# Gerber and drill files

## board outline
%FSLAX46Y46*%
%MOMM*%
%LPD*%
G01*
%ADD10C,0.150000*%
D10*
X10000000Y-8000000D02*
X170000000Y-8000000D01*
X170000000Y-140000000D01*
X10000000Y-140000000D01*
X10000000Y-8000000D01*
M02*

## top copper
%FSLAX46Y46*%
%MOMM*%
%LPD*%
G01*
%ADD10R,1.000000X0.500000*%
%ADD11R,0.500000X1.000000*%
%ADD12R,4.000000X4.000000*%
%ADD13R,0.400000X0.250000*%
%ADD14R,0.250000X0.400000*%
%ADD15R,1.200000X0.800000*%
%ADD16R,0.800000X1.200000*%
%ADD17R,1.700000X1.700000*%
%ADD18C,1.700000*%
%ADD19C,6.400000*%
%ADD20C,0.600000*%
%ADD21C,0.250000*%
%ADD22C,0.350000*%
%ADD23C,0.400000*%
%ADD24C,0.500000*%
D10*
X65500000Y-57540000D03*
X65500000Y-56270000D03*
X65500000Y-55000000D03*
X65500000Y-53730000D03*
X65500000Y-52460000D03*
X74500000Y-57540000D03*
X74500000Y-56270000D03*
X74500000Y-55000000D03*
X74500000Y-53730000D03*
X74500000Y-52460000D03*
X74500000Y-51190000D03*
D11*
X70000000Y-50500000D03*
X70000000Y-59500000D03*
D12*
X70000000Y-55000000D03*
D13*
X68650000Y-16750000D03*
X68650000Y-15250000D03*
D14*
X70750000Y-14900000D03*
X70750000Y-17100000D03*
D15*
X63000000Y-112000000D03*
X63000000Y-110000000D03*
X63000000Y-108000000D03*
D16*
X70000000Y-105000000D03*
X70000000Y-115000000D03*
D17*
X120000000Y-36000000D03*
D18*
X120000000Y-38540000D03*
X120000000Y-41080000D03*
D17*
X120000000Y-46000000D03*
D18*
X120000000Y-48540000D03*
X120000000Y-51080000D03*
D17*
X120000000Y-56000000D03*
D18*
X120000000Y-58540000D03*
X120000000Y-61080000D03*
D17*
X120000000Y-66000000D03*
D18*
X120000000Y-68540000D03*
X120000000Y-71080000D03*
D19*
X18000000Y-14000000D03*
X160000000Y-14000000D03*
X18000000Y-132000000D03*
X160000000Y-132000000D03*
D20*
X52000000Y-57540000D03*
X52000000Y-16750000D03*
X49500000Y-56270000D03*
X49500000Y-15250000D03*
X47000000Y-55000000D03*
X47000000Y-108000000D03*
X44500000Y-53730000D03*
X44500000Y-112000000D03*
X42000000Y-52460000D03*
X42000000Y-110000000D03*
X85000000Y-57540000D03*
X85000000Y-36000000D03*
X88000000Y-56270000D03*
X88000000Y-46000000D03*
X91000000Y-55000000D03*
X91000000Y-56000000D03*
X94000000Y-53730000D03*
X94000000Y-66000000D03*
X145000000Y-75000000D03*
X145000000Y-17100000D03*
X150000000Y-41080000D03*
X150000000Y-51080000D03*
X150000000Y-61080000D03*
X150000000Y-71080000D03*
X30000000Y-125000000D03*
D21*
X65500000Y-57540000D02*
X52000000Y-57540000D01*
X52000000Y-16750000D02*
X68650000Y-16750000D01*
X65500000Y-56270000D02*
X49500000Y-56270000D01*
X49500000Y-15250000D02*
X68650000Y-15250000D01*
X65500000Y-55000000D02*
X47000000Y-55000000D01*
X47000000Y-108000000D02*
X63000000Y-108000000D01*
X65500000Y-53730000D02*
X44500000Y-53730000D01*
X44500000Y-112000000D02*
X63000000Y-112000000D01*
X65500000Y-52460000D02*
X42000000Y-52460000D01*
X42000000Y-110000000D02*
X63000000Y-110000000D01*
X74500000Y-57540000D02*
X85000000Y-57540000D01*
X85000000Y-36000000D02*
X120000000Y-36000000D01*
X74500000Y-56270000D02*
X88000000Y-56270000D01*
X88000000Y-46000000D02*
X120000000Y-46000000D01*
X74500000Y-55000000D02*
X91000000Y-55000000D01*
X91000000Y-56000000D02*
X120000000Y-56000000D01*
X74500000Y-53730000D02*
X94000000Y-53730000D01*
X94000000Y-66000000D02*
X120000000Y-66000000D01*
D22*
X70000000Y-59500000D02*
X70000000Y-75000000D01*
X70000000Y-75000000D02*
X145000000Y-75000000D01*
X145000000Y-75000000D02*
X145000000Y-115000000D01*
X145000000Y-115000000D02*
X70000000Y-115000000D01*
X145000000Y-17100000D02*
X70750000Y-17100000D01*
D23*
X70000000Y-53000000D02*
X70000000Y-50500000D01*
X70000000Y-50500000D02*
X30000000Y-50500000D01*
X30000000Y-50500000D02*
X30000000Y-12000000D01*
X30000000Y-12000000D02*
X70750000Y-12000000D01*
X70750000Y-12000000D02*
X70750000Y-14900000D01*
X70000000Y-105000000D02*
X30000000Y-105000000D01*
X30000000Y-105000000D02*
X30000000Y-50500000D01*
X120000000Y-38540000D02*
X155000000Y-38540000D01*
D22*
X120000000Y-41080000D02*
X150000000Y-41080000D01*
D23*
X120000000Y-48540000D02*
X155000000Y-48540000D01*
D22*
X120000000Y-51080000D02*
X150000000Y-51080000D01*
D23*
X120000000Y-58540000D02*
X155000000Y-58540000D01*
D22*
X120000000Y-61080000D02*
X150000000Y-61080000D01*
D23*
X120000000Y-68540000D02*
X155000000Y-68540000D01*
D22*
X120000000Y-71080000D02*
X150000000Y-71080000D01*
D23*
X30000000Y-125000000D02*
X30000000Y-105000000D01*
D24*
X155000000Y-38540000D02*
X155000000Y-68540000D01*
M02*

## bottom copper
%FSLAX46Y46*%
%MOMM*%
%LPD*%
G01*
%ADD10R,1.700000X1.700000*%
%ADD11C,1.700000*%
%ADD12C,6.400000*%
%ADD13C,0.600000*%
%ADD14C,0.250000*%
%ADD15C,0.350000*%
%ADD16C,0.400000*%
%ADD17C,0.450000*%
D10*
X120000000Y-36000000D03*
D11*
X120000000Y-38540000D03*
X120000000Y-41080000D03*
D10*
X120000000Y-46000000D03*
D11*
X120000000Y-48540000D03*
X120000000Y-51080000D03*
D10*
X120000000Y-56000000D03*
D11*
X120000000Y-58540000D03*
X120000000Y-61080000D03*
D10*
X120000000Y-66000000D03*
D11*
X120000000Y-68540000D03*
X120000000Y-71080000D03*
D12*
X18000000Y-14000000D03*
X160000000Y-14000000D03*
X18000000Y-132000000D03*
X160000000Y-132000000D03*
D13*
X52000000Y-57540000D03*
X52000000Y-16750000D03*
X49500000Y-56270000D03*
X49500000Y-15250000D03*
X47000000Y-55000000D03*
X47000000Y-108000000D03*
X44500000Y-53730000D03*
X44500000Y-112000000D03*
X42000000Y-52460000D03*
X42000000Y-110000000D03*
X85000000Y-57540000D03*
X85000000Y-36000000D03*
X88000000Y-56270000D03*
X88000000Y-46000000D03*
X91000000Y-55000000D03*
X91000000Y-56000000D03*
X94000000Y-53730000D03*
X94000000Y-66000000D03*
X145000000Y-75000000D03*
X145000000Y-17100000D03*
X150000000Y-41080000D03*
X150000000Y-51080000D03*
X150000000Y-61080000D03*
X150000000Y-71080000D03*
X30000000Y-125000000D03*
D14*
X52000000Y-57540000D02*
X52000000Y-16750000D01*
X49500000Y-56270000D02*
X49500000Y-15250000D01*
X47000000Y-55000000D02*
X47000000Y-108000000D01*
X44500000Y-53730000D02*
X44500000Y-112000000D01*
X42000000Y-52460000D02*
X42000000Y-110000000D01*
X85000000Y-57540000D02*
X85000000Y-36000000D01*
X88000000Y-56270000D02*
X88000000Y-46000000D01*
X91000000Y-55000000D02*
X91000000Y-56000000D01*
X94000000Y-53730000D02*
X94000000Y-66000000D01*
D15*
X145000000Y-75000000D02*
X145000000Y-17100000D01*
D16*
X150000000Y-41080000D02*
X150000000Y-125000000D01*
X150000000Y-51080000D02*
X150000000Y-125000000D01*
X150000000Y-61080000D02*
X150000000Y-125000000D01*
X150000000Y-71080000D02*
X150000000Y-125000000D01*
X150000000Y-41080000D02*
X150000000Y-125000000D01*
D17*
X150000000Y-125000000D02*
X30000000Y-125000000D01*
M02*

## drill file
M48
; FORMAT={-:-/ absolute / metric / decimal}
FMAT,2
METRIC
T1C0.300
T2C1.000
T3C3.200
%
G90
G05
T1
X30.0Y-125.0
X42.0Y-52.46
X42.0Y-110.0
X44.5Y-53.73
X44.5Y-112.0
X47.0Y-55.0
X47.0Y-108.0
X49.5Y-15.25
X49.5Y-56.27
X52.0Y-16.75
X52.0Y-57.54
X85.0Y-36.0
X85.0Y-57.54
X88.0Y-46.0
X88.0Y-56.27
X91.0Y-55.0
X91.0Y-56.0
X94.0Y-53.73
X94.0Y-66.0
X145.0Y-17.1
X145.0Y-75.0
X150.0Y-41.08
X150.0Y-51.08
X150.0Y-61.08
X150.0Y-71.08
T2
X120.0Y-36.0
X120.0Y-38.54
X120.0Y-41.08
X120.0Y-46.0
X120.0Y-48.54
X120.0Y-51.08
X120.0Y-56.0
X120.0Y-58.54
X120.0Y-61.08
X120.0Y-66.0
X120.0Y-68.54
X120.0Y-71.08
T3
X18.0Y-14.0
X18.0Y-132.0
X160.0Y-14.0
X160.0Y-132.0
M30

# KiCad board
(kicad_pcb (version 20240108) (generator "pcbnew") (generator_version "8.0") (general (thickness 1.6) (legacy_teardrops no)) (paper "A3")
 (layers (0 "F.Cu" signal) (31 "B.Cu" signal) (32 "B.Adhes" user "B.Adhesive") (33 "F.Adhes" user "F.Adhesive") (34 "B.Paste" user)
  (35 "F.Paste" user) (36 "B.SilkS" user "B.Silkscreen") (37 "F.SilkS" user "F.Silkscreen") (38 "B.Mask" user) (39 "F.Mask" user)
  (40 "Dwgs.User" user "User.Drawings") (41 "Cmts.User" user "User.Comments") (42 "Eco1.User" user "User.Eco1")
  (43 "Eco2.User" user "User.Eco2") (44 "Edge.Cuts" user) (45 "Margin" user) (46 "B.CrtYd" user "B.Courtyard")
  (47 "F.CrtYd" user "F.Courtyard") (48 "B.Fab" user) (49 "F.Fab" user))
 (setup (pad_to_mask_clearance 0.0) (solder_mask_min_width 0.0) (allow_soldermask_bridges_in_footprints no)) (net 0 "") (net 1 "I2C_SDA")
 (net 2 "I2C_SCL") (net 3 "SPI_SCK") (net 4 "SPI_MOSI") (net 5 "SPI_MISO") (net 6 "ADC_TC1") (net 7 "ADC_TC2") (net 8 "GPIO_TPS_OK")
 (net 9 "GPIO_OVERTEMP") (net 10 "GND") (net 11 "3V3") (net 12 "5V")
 (gr_rect (start 10 8) (end 170 140) (stroke (width 0.15) (type solid)) (fill none) (layer "Edge.Cuts"))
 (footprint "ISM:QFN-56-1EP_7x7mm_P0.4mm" (layer "F.Cu") (at 70 55)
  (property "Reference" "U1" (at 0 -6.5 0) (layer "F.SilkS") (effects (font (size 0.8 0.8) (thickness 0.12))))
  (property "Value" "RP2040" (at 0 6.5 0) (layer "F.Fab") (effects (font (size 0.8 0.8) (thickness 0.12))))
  (pad "1" smd rect (at -4.5 2.54) (size 1.0 0.5) (layers "F.Cu" "F.Paste" "F.Mask") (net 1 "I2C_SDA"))
  (pad "2" smd rect (at -4.5 1.27) (size 1.0 0.5) (layers "F.Cu" "F.Paste" "F.Mask") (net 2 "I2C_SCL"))
  (pad "3" smd rect (at -4.5 0) (size 1.0 0.5) (layers "F.Cu" "F.Paste" "F.Mask") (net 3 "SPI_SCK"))
  (pad "4" smd rect (at -4.5 -1.27) (size 1.0 0.5) (layers "F.Cu" "F.Paste" "F.Mask") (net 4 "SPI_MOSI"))
  (pad "5" smd rect (at -4.5 -2.54) (size 1.0 0.5) (layers "F.Cu" "F.Paste" "F.Mask") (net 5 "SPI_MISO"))
  (pad "6" smd rect (at 4.5 2.54) (size 1.0 0.5) (layers "F.Cu" "F.Paste" "F.Mask") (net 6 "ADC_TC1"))
  (pad "7" smd rect (at 4.5 1.27) (size 1.0 0.5) (layers "F.Cu" "F.Paste" "F.Mask") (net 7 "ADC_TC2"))
  (pad "8" smd rect (at 4.5 0) (size 1.0 0.5) (layers "F.Cu" "F.Paste" "F.Mask") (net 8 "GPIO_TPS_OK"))
  (pad "9" smd rect (at 4.5 -1.27) (size 1.0 0.5) (layers "F.Cu" "F.Paste" "F.Mask") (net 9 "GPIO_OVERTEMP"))
  (pad "12" smd rect (at 4.5 -2.54) (size 1.0 0.5) (layers "F.Cu" "F.Paste" "F.Mask"))
  (pad "13" smd rect (at 4.5 -3.81) (size 1.0 0.5) (layers "F.Cu" "F.Paste" "F.Mask"))
  (pad "10" smd rect (at 0 -4.5) (size 0.5 1.0) (layers "F.Cu" "F.Paste" "F.Mask") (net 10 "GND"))
  (pad "11" smd rect (at 0 4.5) (size 0.5 1.0) (layers "F.Cu" "F.Paste" "F.Mask") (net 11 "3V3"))
  (pad "EP" smd rect (at 0 0) (size 4 4) (layers "F.Cu" "F.Paste" "F.Mask") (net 10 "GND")))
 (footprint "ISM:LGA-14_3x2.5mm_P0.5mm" (layer "F.Cu") (at 70 16)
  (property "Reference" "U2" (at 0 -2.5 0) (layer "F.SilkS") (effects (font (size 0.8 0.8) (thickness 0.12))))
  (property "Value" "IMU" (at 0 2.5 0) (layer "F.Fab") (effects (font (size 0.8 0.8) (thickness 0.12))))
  (pad "1" smd rect (at -1.35 0.75) (size 0.4 0.25) (layers "F.Cu" "F.Paste" "F.Mask") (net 1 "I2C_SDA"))
  (pad "2" smd rect (at -1.35 -0.75) (size 0.4 0.25) (layers "F.Cu" "F.Paste" "F.Mask") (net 2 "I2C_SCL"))
  (pad "3" smd rect (at 0.75 -1.1) (size 0.25 0.4) (layers "F.Cu" "F.Paste" "F.Mask") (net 10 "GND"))
  (pad "4" smd rect (at 0.75 1.1) (size 0.25 0.4) (layers "F.Cu" "F.Paste" "F.Mask") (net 11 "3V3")))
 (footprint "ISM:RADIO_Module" (layer "F.Cu") (at 70 110)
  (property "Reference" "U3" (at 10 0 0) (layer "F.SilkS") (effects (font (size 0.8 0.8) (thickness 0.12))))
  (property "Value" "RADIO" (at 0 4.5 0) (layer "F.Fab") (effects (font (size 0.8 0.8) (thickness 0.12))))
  (pad "1" smd rect (at -7 2) (size 1.2 0.8) (layers "F.Cu" "F.Paste" "F.Mask") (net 4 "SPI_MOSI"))
  (pad "2" smd rect (at -7 0) (size 1.2 0.8) (layers "F.Cu" "F.Paste" "F.Mask") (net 5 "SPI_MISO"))
  (pad "3" smd rect (at -7 -2) (size 1.2 0.8) (layers "F.Cu" "F.Paste" "F.Mask") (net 3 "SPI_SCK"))
  (pad "4" smd rect (at 0 -5) (size 0.8 1.2) (layers "F.Cu" "F.Paste" "F.Mask") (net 10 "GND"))
  (pad "5" smd rect (at 0 5) (size 0.8 1.2) (layers "F.Cu" "F.Paste" "F.Mask") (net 11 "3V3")))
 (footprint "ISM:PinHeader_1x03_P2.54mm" (layer "F.Cu") (at 120 36)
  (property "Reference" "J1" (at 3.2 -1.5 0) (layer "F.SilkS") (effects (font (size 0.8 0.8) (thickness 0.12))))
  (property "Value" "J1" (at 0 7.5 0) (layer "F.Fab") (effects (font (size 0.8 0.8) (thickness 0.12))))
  (pad "1" thru_hole rect (at 0 0) (size 1.7 1.7) (drill 1.0) (layers "*.Cu" "*.Mask") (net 6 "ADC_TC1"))
  (pad "2" thru_hole circle (at 0 2.54) (size 1.7 1.7) (drill 1.0) (layers "*.Cu" "*.Mask") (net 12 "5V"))
  (pad "3" thru_hole circle (at 0 5.08) (size 1.7 1.7) (drill 1.0) (layers "*.Cu" "*.Mask") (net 10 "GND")))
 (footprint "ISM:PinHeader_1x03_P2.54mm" (layer "F.Cu") (at 120 46)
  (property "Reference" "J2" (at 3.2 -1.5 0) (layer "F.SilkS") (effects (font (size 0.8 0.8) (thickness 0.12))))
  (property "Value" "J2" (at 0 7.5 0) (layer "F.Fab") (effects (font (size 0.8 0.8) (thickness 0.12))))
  (pad "1" thru_hole rect (at 0 0) (size 1.7 1.7) (drill 1.0) (layers "*.Cu" "*.Mask") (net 7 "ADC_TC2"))
  (pad "2" thru_hole circle (at 0 2.54) (size 1.7 1.7) (drill 1.0) (layers "*.Cu" "*.Mask") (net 12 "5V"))
  (pad "3" thru_hole circle (at 0 5.08) (size 1.7 1.7) (drill 1.0) (layers "*.Cu" "*.Mask") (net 10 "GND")))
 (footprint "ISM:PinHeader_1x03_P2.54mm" (layer "F.Cu") (at 120 56)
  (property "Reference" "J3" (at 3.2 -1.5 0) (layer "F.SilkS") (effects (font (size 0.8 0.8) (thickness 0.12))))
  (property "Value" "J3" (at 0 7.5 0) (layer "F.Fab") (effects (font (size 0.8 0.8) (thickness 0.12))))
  (pad "1" thru_hole rect (at 0 0) (size 1.7 1.7) (drill 1.0) (layers "*.Cu" "*.Mask") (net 8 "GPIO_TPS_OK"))
  (pad "2" thru_hole circle (at 0 2.54) (size 1.7 1.7) (drill 1.0) (layers "*.Cu" "*.Mask") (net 12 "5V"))
  (pad "3" thru_hole circle (at 0 5.08) (size 1.7 1.7) (drill 1.0) (layers "*.Cu" "*.Mask") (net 10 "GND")))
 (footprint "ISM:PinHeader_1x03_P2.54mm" (layer "F.Cu") (at 120 66)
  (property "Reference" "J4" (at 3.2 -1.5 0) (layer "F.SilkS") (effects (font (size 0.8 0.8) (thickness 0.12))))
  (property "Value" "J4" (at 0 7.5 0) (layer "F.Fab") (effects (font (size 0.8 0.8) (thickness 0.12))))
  (pad "1" thru_hole rect (at 0 0) (size 1.7 1.7) (drill 1.0) (layers "*.Cu" "*.Mask") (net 9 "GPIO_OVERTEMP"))
  (pad "2" thru_hole circle (at 0 2.54) (size 1.7 1.7) (drill 1.0) (layers "*.Cu" "*.Mask") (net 12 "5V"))
  (pad "3" thru_hole circle (at 0 5.08) (size 1.7 1.7) (drill 1.0) (layers "*.Cu" "*.Mask") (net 10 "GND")))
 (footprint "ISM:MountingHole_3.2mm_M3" (layer "F.Cu") (at 18 14)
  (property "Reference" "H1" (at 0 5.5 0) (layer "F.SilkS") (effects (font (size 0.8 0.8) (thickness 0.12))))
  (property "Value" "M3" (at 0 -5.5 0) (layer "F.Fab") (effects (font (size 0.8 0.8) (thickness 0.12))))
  (pad "" thru_hole circle (at 0 0) (size 6.4 6.4) (drill 3.2) (layers "*.Cu" "*.Mask")))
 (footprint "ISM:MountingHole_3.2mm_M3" (layer "F.Cu") (at 160 14)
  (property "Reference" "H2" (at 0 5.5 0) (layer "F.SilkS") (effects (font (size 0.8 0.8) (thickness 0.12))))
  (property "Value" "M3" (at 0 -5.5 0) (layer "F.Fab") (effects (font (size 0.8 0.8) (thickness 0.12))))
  (pad "" thru_hole circle (at 0 0) (size 6.4 6.4) (drill 3.2) (layers "*.Cu" "*.Mask")))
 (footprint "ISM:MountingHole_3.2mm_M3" (layer "F.Cu") (at 18 132)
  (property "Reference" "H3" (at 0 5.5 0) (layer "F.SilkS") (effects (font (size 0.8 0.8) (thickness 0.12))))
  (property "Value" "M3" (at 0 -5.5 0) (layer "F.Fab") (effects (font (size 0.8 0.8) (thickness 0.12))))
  (pad "" thru_hole circle (at 0 0) (size 6.4 6.4) (drill 3.2) (layers "*.Cu" "*.Mask")))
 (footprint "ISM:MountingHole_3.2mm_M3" (layer "F.Cu") (at 160 132)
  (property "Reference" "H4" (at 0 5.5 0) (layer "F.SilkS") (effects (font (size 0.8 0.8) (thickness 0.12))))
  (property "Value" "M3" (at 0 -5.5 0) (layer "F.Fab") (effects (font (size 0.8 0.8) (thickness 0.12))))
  (pad "" thru_hole circle (at 0 0) (size 6.4 6.4) (drill 3.2) (layers "*.Cu" "*.Mask")))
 (segment (start 65.5 57.54) (end 52.0 57.54) (width 0.25) (layer "F.Cu") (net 1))
 (segment (start 52.0 57.54) (end 52.0 16.75) (width 0.25) (layer "B.Cu") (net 1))
 (segment (start 52.0 16.75) (end 68.65 16.75) (width 0.25) (layer "F.Cu") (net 1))
 (segment (start 65.5 56.27) (end 49.5 56.27) (width 0.25) (layer "F.Cu") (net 2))
 (segment (start 49.5 56.27) (end 49.5 15.25) (width 0.25) (layer "B.Cu") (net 2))
 (segment (start 49.5 15.25) (end 68.65 15.25) (width 0.25) (layer "F.Cu") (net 2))
 (segment (start 65.5 55) (end 47.0 55) (width 0.25) (layer "F.Cu") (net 3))
 (segment (start 47.0 55) (end 47.0 108) (width 0.25) (layer "B.Cu") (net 3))
 (segment (start 47.0 108) (end 63 108) (width 0.25) (layer "F.Cu") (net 3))
 (segment (start 65.5 53.73) (end 44.5 53.73) (width 0.25) (layer "F.Cu") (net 4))
 (segment (start 44.5 53.73) (end 44.5 112) (width 0.25) (layer "B.Cu") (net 4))
 (segment (start 44.5 112) (end 63 112) (width 0.25) (layer "F.Cu") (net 4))
 (segment (start 65.5 52.46) (end 42.0 52.46) (width 0.25) (layer "F.Cu") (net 5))
 (segment (start 42.0 52.46) (end 42.0 110) (width 0.25) (layer "B.Cu") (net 5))
 (segment (start 42.0 110) (end 63 110) (width 0.25) (layer "F.Cu") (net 5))
 (segment (start 74.5 57.54) (end 85 57.54) (width 0.25) (layer "F.Cu") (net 6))
 (segment (start 85 57.54) (end 85 36) (width 0.25) (layer "B.Cu") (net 6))
 (segment (start 85 36) (end 120 36) (width 0.25) (layer "F.Cu") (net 6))
 (segment (start 74.5 56.27) (end 88 56.27) (width 0.25) (layer "F.Cu") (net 7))
 (segment (start 88 56.27) (end 88 46) (width 0.25) (layer "B.Cu") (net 7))
 (segment (start 88 46) (end 120 46) (width 0.25) (layer "F.Cu") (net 7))
 (segment (start 74.5 55) (end 91 55) (width 0.25) (layer "F.Cu") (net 8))
 (segment (start 91 55) (end 91 56) (width 0.25) (layer "B.Cu") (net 8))
 (segment (start 91 56) (end 120 56) (width 0.25) (layer "F.Cu") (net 8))
 (segment (start 74.5 53.73) (end 94 53.73) (width 0.25) (layer "F.Cu") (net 9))
 (segment (start 94 53.73) (end 94 66) (width 0.25) (layer "B.Cu") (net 9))
 (segment (start 94 66) (end 120 66) (width 0.25) (layer "F.Cu") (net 9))
 (segment (start 70 59.5) (end 70 75) (width 0.35) (layer "F.Cu") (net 11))
 (segment (start 70 75) (end 145 75) (width 0.35) (layer "F.Cu") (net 11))
 (segment (start 145 75) (end 145 115) (width 0.35) (layer "F.Cu") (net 11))
 (segment (start 145 115) (end 70 115) (width 0.35) (layer "F.Cu") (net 11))
 (segment (start 145 75) (end 145 17.1) (width 0.35) (layer "B.Cu") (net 11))
 (segment (start 145 17.1) (end 70.75 17.1) (width 0.35) (layer "F.Cu") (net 11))
 (segment (start 70 53) (end 70 50.5) (width 0.4) (layer "F.Cu") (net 10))
 (segment (start 70 50.5) (end 30 50.5) (width 0.4) (layer "F.Cu") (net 10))
 (segment (start 30 50.5) (end 30 12) (width 0.4) (layer "F.Cu") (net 10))
 (segment (start 30 12) (end 70.75 12) (width 0.4) (layer "F.Cu") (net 10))
 (segment (start 70.75 12) (end 70.75 14.9) (width 0.4) (layer "F.Cu") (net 10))
 (segment (start 70 105) (end 30 105) (width 0.4) (layer "F.Cu") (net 10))
 (segment (start 30 105) (end 30 50.5) (width 0.4) (layer "F.Cu") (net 10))
 (segment (start 120 38.54) (end 155 38.54) (width 0.4) (layer "F.Cu") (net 12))
 (segment (start 120 41.08) (end 150 41.08) (width 0.35) (layer "F.Cu") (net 10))
 (segment (start 150 41.08) (end 150 125) (width 0.4) (layer "B.Cu") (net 10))
 (segment (start 120 48.54) (end 155 48.54) (width 0.4) (layer "F.Cu") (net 12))
 (segment (start 120 51.08) (end 150 51.08) (width 0.35) (layer "F.Cu") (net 10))
 (segment (start 150 51.08) (end 150 125) (width 0.4) (layer "B.Cu") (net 10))
 (segment (start 120 58.54) (end 155 58.54) (width 0.4) (layer "F.Cu") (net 12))
 (segment (start 120 61.08) (end 150 61.08) (width 0.35) (layer "F.Cu") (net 10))
 (segment (start 150 61.08) (end 150 125) (width 0.4) (layer "B.Cu") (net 10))
 (segment (start 120 68.54) (end 155 68.54) (width 0.4) (layer "F.Cu") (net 12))
 (segment (start 120 71.08) (end 150 71.08) (width 0.35) (layer "F.Cu") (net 10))
 (segment (start 150 71.08) (end 150 125) (width 0.4) (layer "B.Cu") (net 10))
 (segment (start 150 41.08) (end 150 125) (width 0.4) (layer "B.Cu") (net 10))
 (segment (start 150 125) (end 30 125) (width 0.45) (layer "B.Cu") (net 10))
 (segment (start 30 125) (end 30 105) (width 0.4) (layer "F.Cu") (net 10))
 (segment (start 155 38.54) (end 155 68.54) (width 0.5) (layer "F.Cu") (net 12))
 (via (at 52.0 57.54) (size 0.6) (drill 0.3) (layers "F.Cu" "B.Cu") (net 1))
 (via (at 52.0 16.75) (size 0.6) (drill 0.3) (layers "F.Cu" "B.Cu") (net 1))
 (via (at 49.5 56.27) (size 0.6) (drill 0.3) (layers "F.Cu" "B.Cu") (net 2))
 (via (at 49.5 15.25) (size 0.6) (drill 0.3) (layers "F.Cu" "B.Cu") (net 2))
 (via (at 47.0 55) (size 0.6) (drill 0.3) (layers "F.Cu" "B.Cu") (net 3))
 (via (at 47.0 108) (size 0.6) (drill 0.3) (layers "F.Cu" "B.Cu") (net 3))
 (via (at 44.5 53.73) (size 0.6) (drill 0.3) (layers "F.Cu" "B.Cu") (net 4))
 (via (at 44.5 112) (size 0.6) (drill 0.3) (layers "F.Cu" "B.Cu") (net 4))
 (via (at 42.0 52.46) (size 0.6) (drill 0.3) (layers "F.Cu" "B.Cu") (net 5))
 (via (at 42.0 110) (size 0.6) (drill 0.3) (layers "F.Cu" "B.Cu") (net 5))
 (via (at 85 57.54) (size 0.6) (drill 0.3) (layers "F.Cu" "B.Cu") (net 6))
 (via (at 85 36) (size 0.6) (drill 0.3) (layers "F.Cu" "B.Cu") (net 6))
 (via (at 88 56.27) (size 0.6) (drill 0.3) (layers "F.Cu" "B.Cu") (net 7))
 (via (at 88 46) (size 0.6) (drill 0.3) (layers "F.Cu" "B.Cu") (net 7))
 (via (at 91 55) (size 0.6) (drill 0.3) (layers "F.Cu" "B.Cu") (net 8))
 (via (at 91 56) (size 0.6) (drill 0.3) (layers "F.Cu" "B.Cu") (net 8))
 (via (at 94 53.73) (size 0.6) (drill 0.3) (layers "F.Cu" "B.Cu") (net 9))
 (via (at 94 66) (size 0.6) (drill 0.3) (layers "F.Cu" "B.Cu") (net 9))
 (via (at 145 75) (size 0.6) (drill 0.3) (layers "F.Cu" "B.Cu") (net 11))
 (via (at 145 17.1) (size 0.6) (drill 0.3) (layers "F.Cu" "B.Cu") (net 11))
 (via (at 150 41.08) (size 0.6) (drill 0.3) (layers "F.Cu" "B.Cu") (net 10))
 (via (at 150 51.08) (size 0.6) (drill 0.3) (layers "F.Cu" "B.Cu") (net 10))
 (via (at 150 61.08) (size 0.6) (drill 0.3) (layers "F.Cu" "B.Cu") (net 10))
 (via (at 150 71.08) (size 0.6) (drill 0.3) (layers "F.Cu" "B.Cu") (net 10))
 (via (at 30 125) (size 0.6) (drill 0.3) (layers "F.Cu" "B.Cu") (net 10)))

